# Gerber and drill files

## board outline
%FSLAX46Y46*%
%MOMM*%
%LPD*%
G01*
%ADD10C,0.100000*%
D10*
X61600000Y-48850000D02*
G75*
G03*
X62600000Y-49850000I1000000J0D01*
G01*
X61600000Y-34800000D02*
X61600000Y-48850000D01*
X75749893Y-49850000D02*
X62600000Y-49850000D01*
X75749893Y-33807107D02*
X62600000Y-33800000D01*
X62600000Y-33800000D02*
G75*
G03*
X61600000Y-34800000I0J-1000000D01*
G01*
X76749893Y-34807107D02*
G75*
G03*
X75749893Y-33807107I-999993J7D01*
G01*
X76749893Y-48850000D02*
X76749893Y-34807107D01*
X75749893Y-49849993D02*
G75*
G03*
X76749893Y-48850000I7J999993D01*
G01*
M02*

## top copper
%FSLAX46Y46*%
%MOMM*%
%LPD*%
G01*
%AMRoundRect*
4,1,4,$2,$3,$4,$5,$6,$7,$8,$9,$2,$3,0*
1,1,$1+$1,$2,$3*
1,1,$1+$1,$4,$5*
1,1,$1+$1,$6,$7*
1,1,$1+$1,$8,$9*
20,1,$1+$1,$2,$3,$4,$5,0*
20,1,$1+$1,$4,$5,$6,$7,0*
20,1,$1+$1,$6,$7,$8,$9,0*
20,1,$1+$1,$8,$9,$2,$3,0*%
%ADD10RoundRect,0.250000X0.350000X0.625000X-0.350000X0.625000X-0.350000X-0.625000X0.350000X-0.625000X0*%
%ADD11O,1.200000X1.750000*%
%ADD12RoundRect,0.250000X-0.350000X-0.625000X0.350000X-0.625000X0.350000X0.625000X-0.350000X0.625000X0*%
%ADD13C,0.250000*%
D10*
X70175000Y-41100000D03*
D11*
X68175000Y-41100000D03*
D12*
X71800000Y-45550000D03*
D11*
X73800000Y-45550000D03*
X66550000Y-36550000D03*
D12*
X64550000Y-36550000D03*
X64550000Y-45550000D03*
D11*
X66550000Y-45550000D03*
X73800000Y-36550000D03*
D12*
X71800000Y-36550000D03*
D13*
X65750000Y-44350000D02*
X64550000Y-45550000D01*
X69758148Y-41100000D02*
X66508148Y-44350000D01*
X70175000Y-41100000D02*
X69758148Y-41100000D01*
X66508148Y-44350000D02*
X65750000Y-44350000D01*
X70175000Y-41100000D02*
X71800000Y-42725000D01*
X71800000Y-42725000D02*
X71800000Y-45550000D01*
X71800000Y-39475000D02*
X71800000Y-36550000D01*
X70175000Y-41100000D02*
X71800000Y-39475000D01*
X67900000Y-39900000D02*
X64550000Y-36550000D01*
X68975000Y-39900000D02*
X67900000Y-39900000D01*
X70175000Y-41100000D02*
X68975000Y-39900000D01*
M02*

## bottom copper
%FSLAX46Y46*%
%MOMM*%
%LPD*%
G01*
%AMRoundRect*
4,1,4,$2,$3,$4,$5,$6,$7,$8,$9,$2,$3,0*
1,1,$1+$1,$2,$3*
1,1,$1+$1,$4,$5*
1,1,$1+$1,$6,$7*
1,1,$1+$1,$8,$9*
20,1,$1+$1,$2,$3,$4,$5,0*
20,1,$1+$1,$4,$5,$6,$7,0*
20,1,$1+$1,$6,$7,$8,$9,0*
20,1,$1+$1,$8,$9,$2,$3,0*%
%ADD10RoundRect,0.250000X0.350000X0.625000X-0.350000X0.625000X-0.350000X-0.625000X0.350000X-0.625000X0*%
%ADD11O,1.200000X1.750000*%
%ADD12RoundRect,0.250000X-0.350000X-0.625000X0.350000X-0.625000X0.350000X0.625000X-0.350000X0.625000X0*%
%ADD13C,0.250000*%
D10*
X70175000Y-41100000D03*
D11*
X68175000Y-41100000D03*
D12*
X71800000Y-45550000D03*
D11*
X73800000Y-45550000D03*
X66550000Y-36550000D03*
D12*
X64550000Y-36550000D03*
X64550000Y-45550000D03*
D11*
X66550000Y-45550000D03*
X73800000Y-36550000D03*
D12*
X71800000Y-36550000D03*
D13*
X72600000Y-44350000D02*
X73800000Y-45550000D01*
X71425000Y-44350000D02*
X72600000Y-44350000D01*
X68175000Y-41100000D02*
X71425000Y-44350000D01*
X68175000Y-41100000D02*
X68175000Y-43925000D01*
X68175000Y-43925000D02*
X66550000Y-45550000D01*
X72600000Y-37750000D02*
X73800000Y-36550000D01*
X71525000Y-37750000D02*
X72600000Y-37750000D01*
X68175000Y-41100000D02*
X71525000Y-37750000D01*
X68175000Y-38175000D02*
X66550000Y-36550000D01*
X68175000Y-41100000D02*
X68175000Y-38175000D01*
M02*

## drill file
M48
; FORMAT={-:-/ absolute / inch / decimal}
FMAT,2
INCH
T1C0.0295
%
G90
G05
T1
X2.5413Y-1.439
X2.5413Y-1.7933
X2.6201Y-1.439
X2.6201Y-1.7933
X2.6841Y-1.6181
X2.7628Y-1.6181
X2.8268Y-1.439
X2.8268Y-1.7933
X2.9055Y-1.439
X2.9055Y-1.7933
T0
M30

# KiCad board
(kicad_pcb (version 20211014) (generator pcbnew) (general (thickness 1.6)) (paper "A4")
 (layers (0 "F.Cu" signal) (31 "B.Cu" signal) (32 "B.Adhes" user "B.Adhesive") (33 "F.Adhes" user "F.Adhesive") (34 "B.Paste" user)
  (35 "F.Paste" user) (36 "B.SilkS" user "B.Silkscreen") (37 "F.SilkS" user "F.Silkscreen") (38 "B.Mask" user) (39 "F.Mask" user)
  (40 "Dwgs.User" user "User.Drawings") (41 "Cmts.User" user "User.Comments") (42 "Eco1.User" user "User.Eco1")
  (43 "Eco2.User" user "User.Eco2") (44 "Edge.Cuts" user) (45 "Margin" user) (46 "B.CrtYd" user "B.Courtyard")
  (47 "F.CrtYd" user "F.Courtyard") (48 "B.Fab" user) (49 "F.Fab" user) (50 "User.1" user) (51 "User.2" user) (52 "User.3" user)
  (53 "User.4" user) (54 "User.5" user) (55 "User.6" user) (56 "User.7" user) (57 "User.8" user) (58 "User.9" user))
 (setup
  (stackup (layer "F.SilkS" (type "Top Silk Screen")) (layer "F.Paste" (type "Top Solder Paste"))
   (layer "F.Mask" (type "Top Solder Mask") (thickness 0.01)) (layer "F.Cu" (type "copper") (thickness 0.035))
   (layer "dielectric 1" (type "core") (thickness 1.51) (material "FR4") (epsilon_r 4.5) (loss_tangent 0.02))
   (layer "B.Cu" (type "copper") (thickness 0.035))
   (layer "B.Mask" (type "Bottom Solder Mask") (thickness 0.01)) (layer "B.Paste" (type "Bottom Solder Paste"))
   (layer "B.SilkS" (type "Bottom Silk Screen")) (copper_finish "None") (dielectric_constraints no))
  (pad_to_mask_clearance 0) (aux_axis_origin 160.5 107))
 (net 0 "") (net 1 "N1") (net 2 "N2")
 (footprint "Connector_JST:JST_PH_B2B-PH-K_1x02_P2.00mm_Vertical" (layer "F.Cu") (at 71.8 45.55)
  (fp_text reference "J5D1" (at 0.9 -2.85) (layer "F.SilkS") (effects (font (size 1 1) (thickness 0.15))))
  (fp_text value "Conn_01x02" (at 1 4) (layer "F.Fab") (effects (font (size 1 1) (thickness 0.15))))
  (pad "1" thru_hole roundrect (at 0 0) (size 1.2 1.75) (drill 0.75) (layers *.Cu *.Mask) (roundrect_rratio 0.2083333333) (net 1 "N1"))
  (pad "2" thru_hole oval (at 2 0) (size 1.2 1.75) (drill 0.75) (layers *.Cu *.Mask) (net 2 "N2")))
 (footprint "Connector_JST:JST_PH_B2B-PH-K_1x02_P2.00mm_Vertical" (layer "F.Cu") (at 64.55 36.55)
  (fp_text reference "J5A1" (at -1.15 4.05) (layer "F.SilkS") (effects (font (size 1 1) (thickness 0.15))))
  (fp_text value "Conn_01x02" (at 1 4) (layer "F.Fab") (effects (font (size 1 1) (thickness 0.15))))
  (pad "1" thru_hole roundrect (at 0 0) (size 1.2 1.75) (drill 0.75) (layers *.Cu *.Mask) (roundrect_rratio 0.2083333333) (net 1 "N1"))
  (pad "2" thru_hole oval (at 2 0) (size 1.2 1.75) (drill 0.75) (layers *.Cu *.Mask) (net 2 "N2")))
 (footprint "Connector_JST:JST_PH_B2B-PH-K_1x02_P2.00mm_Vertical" (layer "F.Cu") (at 64.55 45.55)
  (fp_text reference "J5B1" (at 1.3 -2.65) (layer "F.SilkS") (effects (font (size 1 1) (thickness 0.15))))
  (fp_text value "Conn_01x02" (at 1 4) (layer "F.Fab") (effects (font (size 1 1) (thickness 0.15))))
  (pad "1" thru_hole roundrect (at 0 0) (size 1.2 1.75) (drill 0.75) (layers *.Cu *.Mask) (roundrect_rratio 0.2083333333) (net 1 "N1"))
  (pad "2" thru_hole oval (at 2 0) (size 1.2 1.75) (drill 0.75) (layers *.Cu *.Mask) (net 2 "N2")))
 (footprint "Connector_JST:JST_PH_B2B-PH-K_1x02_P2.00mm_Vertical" (layer "F.Cu") (at 71.8 36.55)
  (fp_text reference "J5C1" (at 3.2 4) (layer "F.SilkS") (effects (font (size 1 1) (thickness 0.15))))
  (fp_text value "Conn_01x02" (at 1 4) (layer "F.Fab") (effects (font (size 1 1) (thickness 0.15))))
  (pad "1" thru_hole roundrect (at 0 0) (size 1.2 1.75) (drill 0.75) (layers *.Cu *.Mask) (roundrect_rratio 0.2083333333) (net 1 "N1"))
  (pad "2" thru_hole oval (at 2 0) (size 1.2 1.75) (drill 0.75) (layers *.Cu *.Mask) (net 2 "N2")))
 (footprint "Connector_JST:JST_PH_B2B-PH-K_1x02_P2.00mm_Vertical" (layer "B.Cu") (at 70.175 41.1 180)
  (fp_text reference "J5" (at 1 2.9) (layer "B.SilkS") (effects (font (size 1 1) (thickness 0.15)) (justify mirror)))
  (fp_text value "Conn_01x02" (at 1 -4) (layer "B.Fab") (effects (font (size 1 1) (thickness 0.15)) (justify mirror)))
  (pad "1" thru_hole roundrect (at 0 0 180) (size 1.2 1.75) (drill 0.75) (layers *.Cu *.Mask) (roundrect_rratio 0.2083333333) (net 1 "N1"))
  (pad "2" thru_hole oval (at 2 0 180) (size 1.2 1.75) (drill 0.75) (layers *.Cu *.Mask) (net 2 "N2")))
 (gr_arc (start 62.6 49.85) (mid 61.892893 49.557107) (end 61.6 48.85) (layer "Edge.Cuts") (width 0.1))
 (gr_line (start 61.6 34.8) (end 61.6 48.85) (layer "Edge.Cuts") (width 0.1))
 (gr_line (start 75.749893 49.85) (end 62.6 49.85) (layer "Edge.Cuts") (width 0.1))
 (gr_line (start 75.749893 33.807107) (end 62.6 33.8) (layer "Edge.Cuts") (width 0.1))
 (gr_arc (start 61.6 34.8) (mid 61.892893 34.092893) (end 62.6 33.8) (layer "Edge.Cuts") (width 0.1))
 (gr_arc (start 75.749893 33.807107) (mid 76.457002 34.099998) (end 76.749893 34.807107) (layer "Edge.Cuts") (width 0.1))
 (gr_line (start 76.749893 48.85) (end 76.749893 34.807107) (layer "Edge.Cuts") (width 0.1))
 (gr_arc (start 76.749893 48.85) (mid 76.456999 49.557104) (end 75.749893 49.85) (layer "Edge.Cuts") (width 0.1))
 (segment (start 71.8 39.475) (end 71.8 36.55) (width 0.25) (layer "F.Cu") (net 1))
 (segment (start 66.508148 44.35) (end 65.75 44.35) (width 0.25) (layer "F.Cu") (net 1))
 (segment (start 68.975 39.9) (end 67.9 39.9) (width 0.25) (layer "F.Cu") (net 1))
 (segment (start 67.9 39.9) (end 64.55 36.55) (width 0.25) (layer "F.Cu") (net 1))
 (segment (start 70.175 41.1) (end 71.8 42.725) (width 0.25) (layer "F.Cu") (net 1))
 (segment (start 69.758148 41.1) (end 66.508148 44.35) (width 0.25) (layer "F.Cu") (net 1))
 (segment (start 70.175 41.1) (end 69.758148 41.1) (width 0.25) (layer "F.Cu") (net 1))
 (segment (start 70.175 41.1) (end 71.8 39.475) (width 0.25) (layer "F.Cu") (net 1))
 (segment (start 65.75 44.35) (end 64.55 45.55) (width 0.25) (layer "F.Cu") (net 1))
 (segment (start 71.8 42.725) (end 71.8 45.55) (width 0.25) (layer "F.Cu") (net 1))
 (segment (start 70.175 41.1) (end 68.975 39.9) (width 0.25) (layer "F.Cu") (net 1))
 (segment (start 71.525 37.75) (end 72.6 37.75) (width 0.25) (layer "B.Cu") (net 2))
 (segment (start 68.175 41.1) (end 68.175 38.175) (width 0.25) (layer "B.Cu") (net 2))
 (segment (start 68.175 41.1) (end 71.425 44.35) (width 0.25) (layer "B.Cu") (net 2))
 (segment (start 68.175 41.1) (end 71.525 37.75) (width 0.25) (layer "B.Cu") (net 2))
 (segment (start 68.175 38.175) (end 66.55 36.55) (width 0.25) (layer "B.Cu") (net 2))
 (segment (start 72.6 44.35) (end 73.8 45.55) (width 0.25) (layer "B.Cu") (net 2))
 (segment (start 68.175 41.1) (end 68.175 43.925) (width 0.25) (layer "B.Cu") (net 2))
 (segment (start 71.425 44.35) (end 72.6 44.35) (width 0.25) (layer "B.Cu") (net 2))
 (segment (start 68.175 43.925) (end 66.55 45.55) (width 0.25) (layer "B.Cu") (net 2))
 (segment (start 72.6 37.75) (end 73.8 36.55) (width 0.25) (layer "B.Cu") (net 2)))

